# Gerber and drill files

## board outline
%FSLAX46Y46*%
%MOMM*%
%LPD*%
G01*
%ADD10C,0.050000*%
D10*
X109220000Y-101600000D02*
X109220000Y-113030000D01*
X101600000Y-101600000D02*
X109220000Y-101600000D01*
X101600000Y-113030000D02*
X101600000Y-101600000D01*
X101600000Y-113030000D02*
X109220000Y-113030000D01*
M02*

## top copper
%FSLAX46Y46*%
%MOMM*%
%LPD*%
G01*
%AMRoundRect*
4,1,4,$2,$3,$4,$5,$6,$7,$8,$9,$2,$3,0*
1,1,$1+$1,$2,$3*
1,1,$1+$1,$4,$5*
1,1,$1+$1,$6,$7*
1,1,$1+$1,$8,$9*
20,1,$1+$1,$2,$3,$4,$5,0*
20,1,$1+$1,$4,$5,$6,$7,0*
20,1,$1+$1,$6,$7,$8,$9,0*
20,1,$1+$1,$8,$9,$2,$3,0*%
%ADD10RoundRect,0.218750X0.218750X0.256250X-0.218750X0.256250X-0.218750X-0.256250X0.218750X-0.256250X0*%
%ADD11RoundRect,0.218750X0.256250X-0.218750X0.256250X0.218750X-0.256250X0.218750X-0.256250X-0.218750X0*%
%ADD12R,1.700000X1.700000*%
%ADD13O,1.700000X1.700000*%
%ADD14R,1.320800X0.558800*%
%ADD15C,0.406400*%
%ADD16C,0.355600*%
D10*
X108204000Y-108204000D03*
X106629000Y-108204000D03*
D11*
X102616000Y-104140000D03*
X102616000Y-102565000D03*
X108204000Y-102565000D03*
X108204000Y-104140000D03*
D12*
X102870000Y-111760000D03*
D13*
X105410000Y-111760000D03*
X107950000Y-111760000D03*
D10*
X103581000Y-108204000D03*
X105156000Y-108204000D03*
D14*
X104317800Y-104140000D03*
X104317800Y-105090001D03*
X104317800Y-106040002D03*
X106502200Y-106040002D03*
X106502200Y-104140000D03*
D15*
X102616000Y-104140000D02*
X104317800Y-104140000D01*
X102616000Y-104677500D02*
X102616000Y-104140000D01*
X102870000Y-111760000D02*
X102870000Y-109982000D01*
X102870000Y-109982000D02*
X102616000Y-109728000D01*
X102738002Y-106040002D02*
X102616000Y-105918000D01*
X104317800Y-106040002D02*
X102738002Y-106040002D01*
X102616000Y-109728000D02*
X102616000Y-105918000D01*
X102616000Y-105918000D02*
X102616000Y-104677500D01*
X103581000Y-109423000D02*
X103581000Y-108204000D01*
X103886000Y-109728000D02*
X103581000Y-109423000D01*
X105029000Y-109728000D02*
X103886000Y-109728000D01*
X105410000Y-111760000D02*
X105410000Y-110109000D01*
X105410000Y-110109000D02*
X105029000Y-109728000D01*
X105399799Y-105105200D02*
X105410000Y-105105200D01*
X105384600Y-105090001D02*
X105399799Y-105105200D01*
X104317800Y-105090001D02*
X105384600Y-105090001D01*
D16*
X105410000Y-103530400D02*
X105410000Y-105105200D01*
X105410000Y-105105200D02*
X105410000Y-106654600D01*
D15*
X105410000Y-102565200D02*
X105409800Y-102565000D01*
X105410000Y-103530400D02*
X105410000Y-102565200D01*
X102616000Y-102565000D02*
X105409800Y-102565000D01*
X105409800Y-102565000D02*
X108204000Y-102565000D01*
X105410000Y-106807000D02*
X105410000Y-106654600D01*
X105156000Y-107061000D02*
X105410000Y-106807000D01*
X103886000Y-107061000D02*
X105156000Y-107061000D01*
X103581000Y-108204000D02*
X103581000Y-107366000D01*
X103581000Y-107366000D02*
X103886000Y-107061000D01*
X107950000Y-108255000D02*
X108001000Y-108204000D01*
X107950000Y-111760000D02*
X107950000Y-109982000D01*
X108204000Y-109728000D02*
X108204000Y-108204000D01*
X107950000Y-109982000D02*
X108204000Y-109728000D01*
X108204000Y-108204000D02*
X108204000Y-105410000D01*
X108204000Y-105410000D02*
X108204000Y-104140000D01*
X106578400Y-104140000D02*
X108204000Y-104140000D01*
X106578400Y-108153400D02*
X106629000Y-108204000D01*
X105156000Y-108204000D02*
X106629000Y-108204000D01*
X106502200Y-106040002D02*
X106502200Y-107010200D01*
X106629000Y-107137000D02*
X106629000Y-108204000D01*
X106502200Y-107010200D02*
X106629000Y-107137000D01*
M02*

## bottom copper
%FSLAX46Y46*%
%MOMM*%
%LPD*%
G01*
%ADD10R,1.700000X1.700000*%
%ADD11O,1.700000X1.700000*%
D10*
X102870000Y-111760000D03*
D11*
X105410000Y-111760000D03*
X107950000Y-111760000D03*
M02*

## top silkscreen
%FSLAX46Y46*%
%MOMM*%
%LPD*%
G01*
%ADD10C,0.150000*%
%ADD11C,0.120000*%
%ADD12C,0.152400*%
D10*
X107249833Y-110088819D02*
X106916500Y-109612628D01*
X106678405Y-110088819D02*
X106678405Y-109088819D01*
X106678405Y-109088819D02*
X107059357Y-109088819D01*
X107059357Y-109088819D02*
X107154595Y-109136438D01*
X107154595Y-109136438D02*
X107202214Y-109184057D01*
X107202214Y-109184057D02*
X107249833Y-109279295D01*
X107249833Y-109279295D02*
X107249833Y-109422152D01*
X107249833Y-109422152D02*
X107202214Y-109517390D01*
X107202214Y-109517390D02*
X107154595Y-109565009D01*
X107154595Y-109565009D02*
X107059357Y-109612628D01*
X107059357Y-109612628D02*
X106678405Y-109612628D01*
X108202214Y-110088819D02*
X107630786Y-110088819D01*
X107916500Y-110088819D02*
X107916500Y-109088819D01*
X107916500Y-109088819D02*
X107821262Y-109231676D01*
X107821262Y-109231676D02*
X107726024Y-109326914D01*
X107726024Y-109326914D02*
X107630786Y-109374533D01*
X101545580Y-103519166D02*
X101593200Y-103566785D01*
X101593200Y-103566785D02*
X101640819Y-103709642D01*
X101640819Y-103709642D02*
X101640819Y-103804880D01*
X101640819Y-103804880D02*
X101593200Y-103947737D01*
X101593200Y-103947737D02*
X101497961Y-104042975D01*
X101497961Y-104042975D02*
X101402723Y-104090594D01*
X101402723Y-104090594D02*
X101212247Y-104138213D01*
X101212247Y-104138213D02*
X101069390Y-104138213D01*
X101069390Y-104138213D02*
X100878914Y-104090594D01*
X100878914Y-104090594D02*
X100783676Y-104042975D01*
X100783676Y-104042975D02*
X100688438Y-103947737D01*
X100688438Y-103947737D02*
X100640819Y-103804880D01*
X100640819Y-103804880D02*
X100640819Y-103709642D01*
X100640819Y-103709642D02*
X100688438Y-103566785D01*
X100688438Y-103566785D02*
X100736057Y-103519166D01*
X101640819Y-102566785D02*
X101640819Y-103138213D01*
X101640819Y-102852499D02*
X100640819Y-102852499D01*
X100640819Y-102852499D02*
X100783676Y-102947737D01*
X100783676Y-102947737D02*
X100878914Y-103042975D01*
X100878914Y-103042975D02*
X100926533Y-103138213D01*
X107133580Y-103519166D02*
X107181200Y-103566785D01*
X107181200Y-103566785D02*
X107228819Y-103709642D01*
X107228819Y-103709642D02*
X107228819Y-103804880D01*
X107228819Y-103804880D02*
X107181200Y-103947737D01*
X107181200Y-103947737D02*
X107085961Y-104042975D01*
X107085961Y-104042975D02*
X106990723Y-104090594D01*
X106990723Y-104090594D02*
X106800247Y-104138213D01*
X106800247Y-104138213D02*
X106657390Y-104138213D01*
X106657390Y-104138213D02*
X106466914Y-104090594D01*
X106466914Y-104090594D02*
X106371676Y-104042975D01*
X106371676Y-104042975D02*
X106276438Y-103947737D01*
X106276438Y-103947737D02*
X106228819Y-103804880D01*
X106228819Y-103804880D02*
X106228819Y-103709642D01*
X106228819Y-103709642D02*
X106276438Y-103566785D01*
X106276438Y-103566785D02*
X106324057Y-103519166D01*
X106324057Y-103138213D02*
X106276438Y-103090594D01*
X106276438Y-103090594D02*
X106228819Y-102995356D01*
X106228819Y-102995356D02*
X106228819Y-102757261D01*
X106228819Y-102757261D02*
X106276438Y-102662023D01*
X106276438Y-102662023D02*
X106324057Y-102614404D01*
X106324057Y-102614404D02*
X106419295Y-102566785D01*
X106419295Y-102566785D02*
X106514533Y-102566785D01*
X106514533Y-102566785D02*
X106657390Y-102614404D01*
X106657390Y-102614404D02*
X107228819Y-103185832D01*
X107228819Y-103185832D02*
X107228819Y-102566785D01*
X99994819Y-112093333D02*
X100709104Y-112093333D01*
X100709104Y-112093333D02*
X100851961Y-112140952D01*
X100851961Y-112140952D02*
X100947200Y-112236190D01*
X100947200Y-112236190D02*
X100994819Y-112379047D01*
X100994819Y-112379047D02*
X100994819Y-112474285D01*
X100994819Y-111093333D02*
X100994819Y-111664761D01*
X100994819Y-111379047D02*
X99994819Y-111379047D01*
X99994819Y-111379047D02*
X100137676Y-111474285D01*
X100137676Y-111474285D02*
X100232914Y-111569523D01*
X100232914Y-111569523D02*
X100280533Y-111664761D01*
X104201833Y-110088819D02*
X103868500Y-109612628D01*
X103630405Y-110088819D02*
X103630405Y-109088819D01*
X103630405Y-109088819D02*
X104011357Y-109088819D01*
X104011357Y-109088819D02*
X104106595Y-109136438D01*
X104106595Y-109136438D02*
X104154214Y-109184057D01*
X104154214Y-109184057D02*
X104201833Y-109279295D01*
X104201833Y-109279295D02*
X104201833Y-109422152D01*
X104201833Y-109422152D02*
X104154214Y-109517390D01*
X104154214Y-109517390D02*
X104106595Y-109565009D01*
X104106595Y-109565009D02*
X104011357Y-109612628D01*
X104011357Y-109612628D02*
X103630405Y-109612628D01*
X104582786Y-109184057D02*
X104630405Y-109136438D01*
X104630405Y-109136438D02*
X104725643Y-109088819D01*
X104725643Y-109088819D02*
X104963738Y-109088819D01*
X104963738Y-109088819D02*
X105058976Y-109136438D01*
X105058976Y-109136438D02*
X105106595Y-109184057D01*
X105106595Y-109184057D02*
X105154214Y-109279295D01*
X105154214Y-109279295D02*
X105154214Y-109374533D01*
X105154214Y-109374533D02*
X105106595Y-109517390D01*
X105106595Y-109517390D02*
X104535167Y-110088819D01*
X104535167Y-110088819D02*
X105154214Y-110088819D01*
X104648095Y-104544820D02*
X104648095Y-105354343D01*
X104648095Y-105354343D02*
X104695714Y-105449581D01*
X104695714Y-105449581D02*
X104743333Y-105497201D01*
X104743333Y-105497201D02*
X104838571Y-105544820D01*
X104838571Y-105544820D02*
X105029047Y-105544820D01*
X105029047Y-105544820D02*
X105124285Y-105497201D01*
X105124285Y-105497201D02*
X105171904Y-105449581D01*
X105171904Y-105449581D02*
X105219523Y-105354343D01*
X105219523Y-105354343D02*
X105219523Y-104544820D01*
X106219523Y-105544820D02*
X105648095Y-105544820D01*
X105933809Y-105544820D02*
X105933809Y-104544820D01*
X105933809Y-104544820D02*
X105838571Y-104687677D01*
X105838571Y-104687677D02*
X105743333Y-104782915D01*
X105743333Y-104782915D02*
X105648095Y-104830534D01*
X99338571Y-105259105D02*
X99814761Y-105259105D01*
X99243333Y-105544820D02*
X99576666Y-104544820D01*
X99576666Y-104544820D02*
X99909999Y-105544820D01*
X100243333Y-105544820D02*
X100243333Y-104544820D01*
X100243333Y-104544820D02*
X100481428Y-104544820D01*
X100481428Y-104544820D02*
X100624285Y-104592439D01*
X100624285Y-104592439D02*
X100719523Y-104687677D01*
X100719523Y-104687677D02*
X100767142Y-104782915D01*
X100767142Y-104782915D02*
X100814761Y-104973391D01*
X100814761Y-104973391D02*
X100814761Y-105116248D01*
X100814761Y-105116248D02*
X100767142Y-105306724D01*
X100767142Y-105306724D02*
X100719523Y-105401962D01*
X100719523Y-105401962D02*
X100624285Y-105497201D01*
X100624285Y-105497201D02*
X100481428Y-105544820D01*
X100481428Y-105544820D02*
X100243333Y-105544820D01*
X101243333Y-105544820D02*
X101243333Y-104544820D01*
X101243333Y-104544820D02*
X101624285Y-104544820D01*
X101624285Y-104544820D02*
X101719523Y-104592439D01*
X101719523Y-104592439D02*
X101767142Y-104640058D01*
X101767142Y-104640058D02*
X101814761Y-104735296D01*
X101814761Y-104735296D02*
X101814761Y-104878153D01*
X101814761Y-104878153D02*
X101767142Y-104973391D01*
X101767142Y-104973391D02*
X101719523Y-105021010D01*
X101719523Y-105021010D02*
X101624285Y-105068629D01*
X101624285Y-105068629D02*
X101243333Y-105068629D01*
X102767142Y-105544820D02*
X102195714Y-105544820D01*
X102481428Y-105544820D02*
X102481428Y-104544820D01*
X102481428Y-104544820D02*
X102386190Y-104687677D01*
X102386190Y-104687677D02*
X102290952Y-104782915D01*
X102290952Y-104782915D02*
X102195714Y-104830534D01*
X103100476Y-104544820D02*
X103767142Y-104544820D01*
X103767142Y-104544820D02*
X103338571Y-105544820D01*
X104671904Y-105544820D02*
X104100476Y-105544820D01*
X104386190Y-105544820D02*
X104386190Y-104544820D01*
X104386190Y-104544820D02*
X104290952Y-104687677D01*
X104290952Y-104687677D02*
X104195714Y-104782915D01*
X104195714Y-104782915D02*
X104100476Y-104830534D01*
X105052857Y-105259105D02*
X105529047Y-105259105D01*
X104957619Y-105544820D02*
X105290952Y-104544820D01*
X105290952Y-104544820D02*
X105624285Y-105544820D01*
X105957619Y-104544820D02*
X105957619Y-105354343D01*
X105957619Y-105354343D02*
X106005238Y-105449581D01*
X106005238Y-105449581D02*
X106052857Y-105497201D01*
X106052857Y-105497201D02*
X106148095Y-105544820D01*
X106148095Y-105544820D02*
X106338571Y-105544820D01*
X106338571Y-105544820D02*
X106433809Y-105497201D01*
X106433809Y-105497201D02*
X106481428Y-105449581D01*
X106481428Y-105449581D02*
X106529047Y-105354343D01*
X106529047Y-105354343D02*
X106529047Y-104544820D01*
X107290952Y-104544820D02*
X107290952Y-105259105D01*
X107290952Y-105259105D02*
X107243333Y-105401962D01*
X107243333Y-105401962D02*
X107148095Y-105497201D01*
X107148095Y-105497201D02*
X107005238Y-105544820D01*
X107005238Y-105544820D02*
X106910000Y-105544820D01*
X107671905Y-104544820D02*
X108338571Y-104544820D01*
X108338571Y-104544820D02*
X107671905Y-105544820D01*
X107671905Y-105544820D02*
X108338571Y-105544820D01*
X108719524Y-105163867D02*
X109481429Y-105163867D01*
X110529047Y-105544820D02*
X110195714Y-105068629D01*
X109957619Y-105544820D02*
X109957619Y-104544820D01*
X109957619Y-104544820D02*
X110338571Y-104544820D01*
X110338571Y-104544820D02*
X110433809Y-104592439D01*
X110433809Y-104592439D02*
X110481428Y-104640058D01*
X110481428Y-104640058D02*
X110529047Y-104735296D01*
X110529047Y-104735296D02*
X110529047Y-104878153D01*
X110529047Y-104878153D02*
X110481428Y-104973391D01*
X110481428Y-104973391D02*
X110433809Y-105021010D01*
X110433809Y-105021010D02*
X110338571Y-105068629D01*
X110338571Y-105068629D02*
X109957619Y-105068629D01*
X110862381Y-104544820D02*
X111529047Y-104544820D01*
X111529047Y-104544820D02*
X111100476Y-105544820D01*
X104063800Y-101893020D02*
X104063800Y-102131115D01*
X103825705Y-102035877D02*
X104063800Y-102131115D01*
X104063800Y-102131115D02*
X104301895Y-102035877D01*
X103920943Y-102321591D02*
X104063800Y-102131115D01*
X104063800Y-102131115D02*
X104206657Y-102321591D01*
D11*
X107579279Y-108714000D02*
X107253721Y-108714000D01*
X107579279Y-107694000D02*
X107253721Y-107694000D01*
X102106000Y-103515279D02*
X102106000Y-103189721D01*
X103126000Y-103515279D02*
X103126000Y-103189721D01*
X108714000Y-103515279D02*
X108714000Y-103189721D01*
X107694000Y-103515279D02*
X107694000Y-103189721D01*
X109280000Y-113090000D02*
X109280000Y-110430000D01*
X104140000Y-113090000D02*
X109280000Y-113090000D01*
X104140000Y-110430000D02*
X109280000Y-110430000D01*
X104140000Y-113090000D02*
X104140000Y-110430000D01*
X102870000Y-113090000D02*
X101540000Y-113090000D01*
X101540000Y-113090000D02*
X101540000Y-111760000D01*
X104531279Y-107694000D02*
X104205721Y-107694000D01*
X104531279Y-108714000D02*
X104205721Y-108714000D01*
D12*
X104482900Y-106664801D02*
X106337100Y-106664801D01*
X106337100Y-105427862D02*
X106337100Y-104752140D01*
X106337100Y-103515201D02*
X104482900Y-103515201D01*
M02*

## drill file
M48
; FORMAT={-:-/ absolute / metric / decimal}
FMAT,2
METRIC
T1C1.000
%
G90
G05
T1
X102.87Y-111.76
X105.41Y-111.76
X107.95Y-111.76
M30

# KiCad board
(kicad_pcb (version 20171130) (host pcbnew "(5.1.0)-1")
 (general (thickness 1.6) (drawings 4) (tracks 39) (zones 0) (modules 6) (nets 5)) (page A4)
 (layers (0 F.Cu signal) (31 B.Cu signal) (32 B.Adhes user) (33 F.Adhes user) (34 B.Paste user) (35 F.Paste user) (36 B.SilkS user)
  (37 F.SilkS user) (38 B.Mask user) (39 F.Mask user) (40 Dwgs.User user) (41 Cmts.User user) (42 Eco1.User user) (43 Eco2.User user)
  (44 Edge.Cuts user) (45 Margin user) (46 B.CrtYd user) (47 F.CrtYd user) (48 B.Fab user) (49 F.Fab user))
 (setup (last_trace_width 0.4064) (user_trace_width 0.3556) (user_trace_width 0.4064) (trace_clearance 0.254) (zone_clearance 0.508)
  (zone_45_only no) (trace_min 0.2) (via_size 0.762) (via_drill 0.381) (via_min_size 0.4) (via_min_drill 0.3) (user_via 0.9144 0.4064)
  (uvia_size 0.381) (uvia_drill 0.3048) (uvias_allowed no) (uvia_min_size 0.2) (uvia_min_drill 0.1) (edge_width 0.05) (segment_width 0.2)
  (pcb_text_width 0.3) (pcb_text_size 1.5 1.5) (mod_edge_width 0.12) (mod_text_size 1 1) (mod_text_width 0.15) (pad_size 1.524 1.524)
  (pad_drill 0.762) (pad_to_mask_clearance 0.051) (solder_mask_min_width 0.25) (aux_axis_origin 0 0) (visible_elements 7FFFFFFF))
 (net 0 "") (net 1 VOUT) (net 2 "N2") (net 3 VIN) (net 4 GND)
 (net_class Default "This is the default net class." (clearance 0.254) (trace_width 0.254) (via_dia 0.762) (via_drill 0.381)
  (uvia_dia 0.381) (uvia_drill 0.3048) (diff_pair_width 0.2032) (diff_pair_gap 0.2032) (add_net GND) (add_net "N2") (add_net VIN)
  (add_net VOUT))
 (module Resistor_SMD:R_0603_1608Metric (layer F.Cu) (at 107.4165 108.204 180)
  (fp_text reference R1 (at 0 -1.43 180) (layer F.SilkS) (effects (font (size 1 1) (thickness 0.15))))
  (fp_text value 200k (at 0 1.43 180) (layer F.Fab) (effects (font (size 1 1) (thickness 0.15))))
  (fp_line (start -0.162779 -0.51) (end 0.162779 -0.51) (layer F.SilkS) (width 0.12))
  (fp_line (start -0.162779 0.51) (end 0.162779 0.51) (layer F.SilkS) (width 0.12))
  (pad 1 smd roundrect (at -0.7875 0 180) (size 0.875 0.95) (layers F.Cu F.Paste F.Mask) (roundrect_rratio 0.25) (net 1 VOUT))
  (pad 2 smd roundrect (at 0.7875 0 180) (size 0.875 0.95) (layers F.Cu F.Paste F.Mask) (roundrect_rratio 0.25) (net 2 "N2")))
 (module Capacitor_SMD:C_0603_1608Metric (layer F.Cu) (at 102.616 103.3525 90)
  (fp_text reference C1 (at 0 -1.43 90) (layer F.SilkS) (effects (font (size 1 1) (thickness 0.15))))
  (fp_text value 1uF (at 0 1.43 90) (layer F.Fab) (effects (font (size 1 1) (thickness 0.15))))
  (fp_line (start -0.162779 -0.51) (end 0.162779 -0.51) (layer F.SilkS) (width 0.12))
  (fp_line (start -0.162779 0.51) (end 0.162779 0.51) (layer F.SilkS) (width 0.12))
  (pad 1 smd roundrect (at -0.7875 0 90) (size 0.875 0.95) (layers F.Cu F.Paste F.Mask) (roundrect_rratio 0.25) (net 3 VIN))
  (pad 2 smd roundrect (at 0.7875 0 90) (size 0.875 0.95) (layers F.Cu F.Paste F.Mask) (roundrect_rratio 0.25) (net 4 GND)))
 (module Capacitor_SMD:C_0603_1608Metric (layer F.Cu) (at 108.204 103.3525 90)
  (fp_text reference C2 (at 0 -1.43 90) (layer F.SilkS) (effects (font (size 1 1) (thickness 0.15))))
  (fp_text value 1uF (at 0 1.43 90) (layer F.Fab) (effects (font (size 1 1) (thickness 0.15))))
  (fp_line (start -0.162779 0.51) (end 0.162779 0.51) (layer F.SilkS) (width 0.12))
  (fp_line (start -0.162779 -0.51) (end 0.162779 -0.51) (layer F.SilkS) (width 0.12))
  (pad 2 smd roundrect (at 0.7875 0 90) (size 0.875 0.95) (layers F.Cu F.Paste F.Mask) (roundrect_rratio 0.25) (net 4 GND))
  (pad 1 smd roundrect (at -0.7875 0 90) (size 0.875 0.95) (layers F.Cu F.Paste F.Mask) (roundrect_rratio 0.25) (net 1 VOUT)))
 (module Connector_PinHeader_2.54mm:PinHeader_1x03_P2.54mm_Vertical (layer F.Cu) (at 102.87 111.76 90)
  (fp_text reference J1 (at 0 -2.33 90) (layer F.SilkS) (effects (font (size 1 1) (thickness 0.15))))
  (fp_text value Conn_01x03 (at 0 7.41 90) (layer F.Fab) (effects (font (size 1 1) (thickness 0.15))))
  (fp_line (start -1.33 6.41) (end 1.33 6.41) (layer F.SilkS) (width 0.12))
  (fp_line (start -1.33 1.27) (end -1.33 6.41) (layer F.SilkS) (width 0.12))
  (fp_line (start 1.33 1.27) (end 1.33 6.41) (layer F.SilkS) (width 0.12))
  (fp_line (start -1.33 1.27) (end 1.33 1.27) (layer F.SilkS) (width 0.12))
  (fp_line (start -1.33 0) (end -1.33 -1.33) (layer F.SilkS) (width 0.12))
  (fp_line (start -1.33 -1.33) (end 0 -1.33) (layer F.SilkS) (width 0.12))
  (pad 1 thru_hole rect (at 0 0 90) (size 1.7 1.7) (drill 1) (layers *.Cu *.Mask) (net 3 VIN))
  (pad 2 thru_hole oval (at 0 2.54 90) (size 1.7 1.7) (drill 1) (layers *.Cu *.Mask) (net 4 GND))
  (pad 3 thru_hole oval (at 0 5.08 90) (size 1.7 1.7) (drill 1) (layers *.Cu *.Mask) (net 1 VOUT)))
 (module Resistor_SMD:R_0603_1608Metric (layer F.Cu) (at 104.3685 108.204 180)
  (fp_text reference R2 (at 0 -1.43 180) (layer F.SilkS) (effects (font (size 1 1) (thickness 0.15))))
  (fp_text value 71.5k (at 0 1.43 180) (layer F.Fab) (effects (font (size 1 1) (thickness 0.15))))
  (fp_line (start -0.162779 0.51) (end 0.162779 0.51) (layer F.SilkS) (width 0.12))
  (fp_line (start -0.162779 -0.51) (end 0.162779 -0.51) (layer F.SilkS) (width 0.12))
  (pad 2 smd roundrect (at 0.7875 0 180) (size 0.875 0.95) (layers F.Cu F.Paste F.Mask) (roundrect_rratio 0.25) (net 4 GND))
  (pad 1 smd roundrect (at -0.7875 0 180) (size 0.875 0.95) (layers F.Cu F.Paste F.Mask) (roundrect_rratio 0.25) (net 2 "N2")))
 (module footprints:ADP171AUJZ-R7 (layer F.Cu) (at 105.41 105.090001)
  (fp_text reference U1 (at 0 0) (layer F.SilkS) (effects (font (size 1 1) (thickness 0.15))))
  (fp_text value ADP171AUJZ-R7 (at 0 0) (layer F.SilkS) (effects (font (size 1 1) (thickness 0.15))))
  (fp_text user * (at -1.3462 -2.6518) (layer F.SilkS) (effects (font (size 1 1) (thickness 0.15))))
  (fp_line (start -0.9271 1.5748) (end 0.9271 1.5748) (layer F.SilkS) (width 0.1524))
  (fp_line (start 0.9271 0.337861) (end 0.9271 -0.337861) (layer F.SilkS) (width 0.1524))
  (fp_line (start 0.9271 -1.5748) (end -0.9271 -1.5748) (layer F.SilkS) (width 0.1524))
  (pad 1 smd rect (at -1.0922 -0.950001) (size 1.3208 0.5588) (layers F.Cu F.Paste F.Mask) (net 3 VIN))
  (pad 2 smd rect (at -1.0922 0) (size 1.3208 0.5588) (layers F.Cu F.Paste F.Mask) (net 4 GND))
  (pad 3 smd rect (at -1.0922 0.950001) (size 1.3208 0.5588) (layers F.Cu F.Paste F.Mask) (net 3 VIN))
  (pad 4 smd rect (at 1.0922 0.950001) (size 1.3208 0.5588) (layers F.Cu F.Paste F.Mask) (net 2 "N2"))
  (pad 5 smd rect (at 1.0922 -0.950001) (size 1.3208 0.5588) (layers F.Cu F.Paste F.Mask) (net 1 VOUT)))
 (gr_line (start 109.22 101.6) (end 109.22 113.03) (layer Edge.Cuts) (width 0.05))
 (gr_line (start 101.6 101.6) (end 109.22 101.6) (layer Edge.Cuts) (width 0.05))
 (gr_line (start 101.6 113.03) (end 101.6 101.6) (layer Edge.Cuts) (width 0.05))
 (gr_line (start 101.6 113.03) (end 109.22 113.03) (layer Edge.Cuts) (width 0.05))
 (segment (start 102.616 104.14) (end 104.3178 104.14) (width 0.4064) (layer F.Cu) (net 3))
 (segment (start 102.616 104.6775) (end 102.616 104.14) (width 0.4064) (layer F.Cu) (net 3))
 (segment (start 102.87 111.76) (end 102.87 109.982) (width 0.4064) (layer F.Cu) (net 3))
 (segment (start 102.87 109.982) (end 102.616 109.728) (width 0.4064) (layer F.Cu) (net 3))
 (segment (start 102.738002 106.040002) (end 102.616 105.918) (width 0.4064) (layer F.Cu) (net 3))
 (segment (start 104.3178 106.040002) (end 102.738002 106.040002) (width 0.4064) (layer F.Cu) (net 3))
 (segment (start 102.616 109.728) (end 102.616 105.918) (width 0.4064) (layer F.Cu) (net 3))
 (segment (start 102.616 105.918) (end 102.616 104.6775) (width 0.4064) (layer F.Cu) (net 3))
 (segment (start 103.581 109.423) (end 103.581 108.204) (width 0.4064) (layer F.Cu) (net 4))
 (segment (start 103.886 109.728) (end 103.581 109.423) (width 0.4064) (layer F.Cu) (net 4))
 (segment (start 105.029 109.728) (end 103.886 109.728) (width 0.4064) (layer F.Cu) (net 4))
 (segment (start 105.41 111.76) (end 105.41 110.109) (width 0.4064) (layer F.Cu) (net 4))
 (segment (start 105.41 110.109) (end 105.029 109.728) (width 0.4064) (layer F.Cu) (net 4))
 (segment (start 105.399799 105.1052) (end 105.41 105.1052) (width 0.4064) (layer F.Cu) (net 4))
 (segment (start 105.3846 105.090001) (end 105.399799 105.1052) (width 0.4064) (layer F.Cu) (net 4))
 (segment (start 104.3178 105.090001) (end 105.3846 105.090001) (width 0.4064) (layer F.Cu) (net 4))
 (segment (start 105.41 103.5304) (end 105.41 105.1052) (width 0.3556) (layer F.Cu) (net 4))
 (segment (start 105.41 105.1052) (end 105.41 106.6546) (width 0.3556) (layer F.Cu) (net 4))
 (segment (start 105.41 102.5652) (end 105.4098 102.565) (width 0.4064) (layer F.Cu) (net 4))
 (segment (start 105.41 103.5304) (end 105.41 102.5652) (width 0.4064) (layer F.Cu) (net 4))
 (segment (start 102.616 102.565) (end 105.4098 102.565) (width 0.4064) (layer F.Cu) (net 4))
 (segment (start 105.4098 102.565) (end 108.204 102.565) (width 0.4064) (layer F.Cu) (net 4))
 (segment (start 105.41 106.807) (end 105.41 106.6546) (width 0.4064) (layer F.Cu) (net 4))
 (segment (start 105.156 107.061) (end 105.41 106.807) (width 0.4064) (layer F.Cu) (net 4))
 (segment (start 103.886 107.061) (end 105.156 107.061) (width 0.4064) (layer F.Cu) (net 4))
 (segment (start 103.581 108.204) (end 103.581 107.366) (width 0.4064) (layer F.Cu) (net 4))
 (segment (start 103.581 107.366) (end 103.886 107.061) (width 0.4064) (layer F.Cu) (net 4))
 (segment (start 107.95 108.255) (end 108.001 108.204) (width 0.4064) (layer F.Cu) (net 1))
 (segment (start 107.95 111.76) (end 107.95 109.982) (width 0.4064) (layer F.Cu) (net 1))
 (segment (start 108.204 109.728) (end 108.204 108.204) (width 0.4064) (layer F.Cu) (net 1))
 (segment (start 107.95 109.982) (end 108.204 109.728) (width 0.4064) (layer F.Cu) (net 1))
 (segment (start 108.204 108.204) (end 108.204 105.41) (width 0.4064) (layer F.Cu) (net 1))
 (segment (start 108.204 105.41) (end 108.204 104.14) (width 0.4064) (layer F.Cu) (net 1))
 (segment (start 106.5784 104.14) (end 108.204 104.14) (width 0.4064) (layer F.Cu) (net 1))
 (segment (start 106.5784 108.1534) (end 106.629 108.204) (width 0.4064) (layer F.Cu) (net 2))
 (segment (start 105.156 108.204) (end 106.629 108.204) (width 0.4064) (layer F.Cu) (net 2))
 (segment (start 106.5022 106.040002) (end 106.5022 107.0102) (width 0.4064) (layer F.Cu) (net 2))
 (segment (start 106.629 107.137) (end 106.629 108.204) (width 0.4064) (layer F.Cu) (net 2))
 (segment (start 106.5022 107.0102) (end 106.629 107.137) (width 0.4064) (layer F.Cu) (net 2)))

